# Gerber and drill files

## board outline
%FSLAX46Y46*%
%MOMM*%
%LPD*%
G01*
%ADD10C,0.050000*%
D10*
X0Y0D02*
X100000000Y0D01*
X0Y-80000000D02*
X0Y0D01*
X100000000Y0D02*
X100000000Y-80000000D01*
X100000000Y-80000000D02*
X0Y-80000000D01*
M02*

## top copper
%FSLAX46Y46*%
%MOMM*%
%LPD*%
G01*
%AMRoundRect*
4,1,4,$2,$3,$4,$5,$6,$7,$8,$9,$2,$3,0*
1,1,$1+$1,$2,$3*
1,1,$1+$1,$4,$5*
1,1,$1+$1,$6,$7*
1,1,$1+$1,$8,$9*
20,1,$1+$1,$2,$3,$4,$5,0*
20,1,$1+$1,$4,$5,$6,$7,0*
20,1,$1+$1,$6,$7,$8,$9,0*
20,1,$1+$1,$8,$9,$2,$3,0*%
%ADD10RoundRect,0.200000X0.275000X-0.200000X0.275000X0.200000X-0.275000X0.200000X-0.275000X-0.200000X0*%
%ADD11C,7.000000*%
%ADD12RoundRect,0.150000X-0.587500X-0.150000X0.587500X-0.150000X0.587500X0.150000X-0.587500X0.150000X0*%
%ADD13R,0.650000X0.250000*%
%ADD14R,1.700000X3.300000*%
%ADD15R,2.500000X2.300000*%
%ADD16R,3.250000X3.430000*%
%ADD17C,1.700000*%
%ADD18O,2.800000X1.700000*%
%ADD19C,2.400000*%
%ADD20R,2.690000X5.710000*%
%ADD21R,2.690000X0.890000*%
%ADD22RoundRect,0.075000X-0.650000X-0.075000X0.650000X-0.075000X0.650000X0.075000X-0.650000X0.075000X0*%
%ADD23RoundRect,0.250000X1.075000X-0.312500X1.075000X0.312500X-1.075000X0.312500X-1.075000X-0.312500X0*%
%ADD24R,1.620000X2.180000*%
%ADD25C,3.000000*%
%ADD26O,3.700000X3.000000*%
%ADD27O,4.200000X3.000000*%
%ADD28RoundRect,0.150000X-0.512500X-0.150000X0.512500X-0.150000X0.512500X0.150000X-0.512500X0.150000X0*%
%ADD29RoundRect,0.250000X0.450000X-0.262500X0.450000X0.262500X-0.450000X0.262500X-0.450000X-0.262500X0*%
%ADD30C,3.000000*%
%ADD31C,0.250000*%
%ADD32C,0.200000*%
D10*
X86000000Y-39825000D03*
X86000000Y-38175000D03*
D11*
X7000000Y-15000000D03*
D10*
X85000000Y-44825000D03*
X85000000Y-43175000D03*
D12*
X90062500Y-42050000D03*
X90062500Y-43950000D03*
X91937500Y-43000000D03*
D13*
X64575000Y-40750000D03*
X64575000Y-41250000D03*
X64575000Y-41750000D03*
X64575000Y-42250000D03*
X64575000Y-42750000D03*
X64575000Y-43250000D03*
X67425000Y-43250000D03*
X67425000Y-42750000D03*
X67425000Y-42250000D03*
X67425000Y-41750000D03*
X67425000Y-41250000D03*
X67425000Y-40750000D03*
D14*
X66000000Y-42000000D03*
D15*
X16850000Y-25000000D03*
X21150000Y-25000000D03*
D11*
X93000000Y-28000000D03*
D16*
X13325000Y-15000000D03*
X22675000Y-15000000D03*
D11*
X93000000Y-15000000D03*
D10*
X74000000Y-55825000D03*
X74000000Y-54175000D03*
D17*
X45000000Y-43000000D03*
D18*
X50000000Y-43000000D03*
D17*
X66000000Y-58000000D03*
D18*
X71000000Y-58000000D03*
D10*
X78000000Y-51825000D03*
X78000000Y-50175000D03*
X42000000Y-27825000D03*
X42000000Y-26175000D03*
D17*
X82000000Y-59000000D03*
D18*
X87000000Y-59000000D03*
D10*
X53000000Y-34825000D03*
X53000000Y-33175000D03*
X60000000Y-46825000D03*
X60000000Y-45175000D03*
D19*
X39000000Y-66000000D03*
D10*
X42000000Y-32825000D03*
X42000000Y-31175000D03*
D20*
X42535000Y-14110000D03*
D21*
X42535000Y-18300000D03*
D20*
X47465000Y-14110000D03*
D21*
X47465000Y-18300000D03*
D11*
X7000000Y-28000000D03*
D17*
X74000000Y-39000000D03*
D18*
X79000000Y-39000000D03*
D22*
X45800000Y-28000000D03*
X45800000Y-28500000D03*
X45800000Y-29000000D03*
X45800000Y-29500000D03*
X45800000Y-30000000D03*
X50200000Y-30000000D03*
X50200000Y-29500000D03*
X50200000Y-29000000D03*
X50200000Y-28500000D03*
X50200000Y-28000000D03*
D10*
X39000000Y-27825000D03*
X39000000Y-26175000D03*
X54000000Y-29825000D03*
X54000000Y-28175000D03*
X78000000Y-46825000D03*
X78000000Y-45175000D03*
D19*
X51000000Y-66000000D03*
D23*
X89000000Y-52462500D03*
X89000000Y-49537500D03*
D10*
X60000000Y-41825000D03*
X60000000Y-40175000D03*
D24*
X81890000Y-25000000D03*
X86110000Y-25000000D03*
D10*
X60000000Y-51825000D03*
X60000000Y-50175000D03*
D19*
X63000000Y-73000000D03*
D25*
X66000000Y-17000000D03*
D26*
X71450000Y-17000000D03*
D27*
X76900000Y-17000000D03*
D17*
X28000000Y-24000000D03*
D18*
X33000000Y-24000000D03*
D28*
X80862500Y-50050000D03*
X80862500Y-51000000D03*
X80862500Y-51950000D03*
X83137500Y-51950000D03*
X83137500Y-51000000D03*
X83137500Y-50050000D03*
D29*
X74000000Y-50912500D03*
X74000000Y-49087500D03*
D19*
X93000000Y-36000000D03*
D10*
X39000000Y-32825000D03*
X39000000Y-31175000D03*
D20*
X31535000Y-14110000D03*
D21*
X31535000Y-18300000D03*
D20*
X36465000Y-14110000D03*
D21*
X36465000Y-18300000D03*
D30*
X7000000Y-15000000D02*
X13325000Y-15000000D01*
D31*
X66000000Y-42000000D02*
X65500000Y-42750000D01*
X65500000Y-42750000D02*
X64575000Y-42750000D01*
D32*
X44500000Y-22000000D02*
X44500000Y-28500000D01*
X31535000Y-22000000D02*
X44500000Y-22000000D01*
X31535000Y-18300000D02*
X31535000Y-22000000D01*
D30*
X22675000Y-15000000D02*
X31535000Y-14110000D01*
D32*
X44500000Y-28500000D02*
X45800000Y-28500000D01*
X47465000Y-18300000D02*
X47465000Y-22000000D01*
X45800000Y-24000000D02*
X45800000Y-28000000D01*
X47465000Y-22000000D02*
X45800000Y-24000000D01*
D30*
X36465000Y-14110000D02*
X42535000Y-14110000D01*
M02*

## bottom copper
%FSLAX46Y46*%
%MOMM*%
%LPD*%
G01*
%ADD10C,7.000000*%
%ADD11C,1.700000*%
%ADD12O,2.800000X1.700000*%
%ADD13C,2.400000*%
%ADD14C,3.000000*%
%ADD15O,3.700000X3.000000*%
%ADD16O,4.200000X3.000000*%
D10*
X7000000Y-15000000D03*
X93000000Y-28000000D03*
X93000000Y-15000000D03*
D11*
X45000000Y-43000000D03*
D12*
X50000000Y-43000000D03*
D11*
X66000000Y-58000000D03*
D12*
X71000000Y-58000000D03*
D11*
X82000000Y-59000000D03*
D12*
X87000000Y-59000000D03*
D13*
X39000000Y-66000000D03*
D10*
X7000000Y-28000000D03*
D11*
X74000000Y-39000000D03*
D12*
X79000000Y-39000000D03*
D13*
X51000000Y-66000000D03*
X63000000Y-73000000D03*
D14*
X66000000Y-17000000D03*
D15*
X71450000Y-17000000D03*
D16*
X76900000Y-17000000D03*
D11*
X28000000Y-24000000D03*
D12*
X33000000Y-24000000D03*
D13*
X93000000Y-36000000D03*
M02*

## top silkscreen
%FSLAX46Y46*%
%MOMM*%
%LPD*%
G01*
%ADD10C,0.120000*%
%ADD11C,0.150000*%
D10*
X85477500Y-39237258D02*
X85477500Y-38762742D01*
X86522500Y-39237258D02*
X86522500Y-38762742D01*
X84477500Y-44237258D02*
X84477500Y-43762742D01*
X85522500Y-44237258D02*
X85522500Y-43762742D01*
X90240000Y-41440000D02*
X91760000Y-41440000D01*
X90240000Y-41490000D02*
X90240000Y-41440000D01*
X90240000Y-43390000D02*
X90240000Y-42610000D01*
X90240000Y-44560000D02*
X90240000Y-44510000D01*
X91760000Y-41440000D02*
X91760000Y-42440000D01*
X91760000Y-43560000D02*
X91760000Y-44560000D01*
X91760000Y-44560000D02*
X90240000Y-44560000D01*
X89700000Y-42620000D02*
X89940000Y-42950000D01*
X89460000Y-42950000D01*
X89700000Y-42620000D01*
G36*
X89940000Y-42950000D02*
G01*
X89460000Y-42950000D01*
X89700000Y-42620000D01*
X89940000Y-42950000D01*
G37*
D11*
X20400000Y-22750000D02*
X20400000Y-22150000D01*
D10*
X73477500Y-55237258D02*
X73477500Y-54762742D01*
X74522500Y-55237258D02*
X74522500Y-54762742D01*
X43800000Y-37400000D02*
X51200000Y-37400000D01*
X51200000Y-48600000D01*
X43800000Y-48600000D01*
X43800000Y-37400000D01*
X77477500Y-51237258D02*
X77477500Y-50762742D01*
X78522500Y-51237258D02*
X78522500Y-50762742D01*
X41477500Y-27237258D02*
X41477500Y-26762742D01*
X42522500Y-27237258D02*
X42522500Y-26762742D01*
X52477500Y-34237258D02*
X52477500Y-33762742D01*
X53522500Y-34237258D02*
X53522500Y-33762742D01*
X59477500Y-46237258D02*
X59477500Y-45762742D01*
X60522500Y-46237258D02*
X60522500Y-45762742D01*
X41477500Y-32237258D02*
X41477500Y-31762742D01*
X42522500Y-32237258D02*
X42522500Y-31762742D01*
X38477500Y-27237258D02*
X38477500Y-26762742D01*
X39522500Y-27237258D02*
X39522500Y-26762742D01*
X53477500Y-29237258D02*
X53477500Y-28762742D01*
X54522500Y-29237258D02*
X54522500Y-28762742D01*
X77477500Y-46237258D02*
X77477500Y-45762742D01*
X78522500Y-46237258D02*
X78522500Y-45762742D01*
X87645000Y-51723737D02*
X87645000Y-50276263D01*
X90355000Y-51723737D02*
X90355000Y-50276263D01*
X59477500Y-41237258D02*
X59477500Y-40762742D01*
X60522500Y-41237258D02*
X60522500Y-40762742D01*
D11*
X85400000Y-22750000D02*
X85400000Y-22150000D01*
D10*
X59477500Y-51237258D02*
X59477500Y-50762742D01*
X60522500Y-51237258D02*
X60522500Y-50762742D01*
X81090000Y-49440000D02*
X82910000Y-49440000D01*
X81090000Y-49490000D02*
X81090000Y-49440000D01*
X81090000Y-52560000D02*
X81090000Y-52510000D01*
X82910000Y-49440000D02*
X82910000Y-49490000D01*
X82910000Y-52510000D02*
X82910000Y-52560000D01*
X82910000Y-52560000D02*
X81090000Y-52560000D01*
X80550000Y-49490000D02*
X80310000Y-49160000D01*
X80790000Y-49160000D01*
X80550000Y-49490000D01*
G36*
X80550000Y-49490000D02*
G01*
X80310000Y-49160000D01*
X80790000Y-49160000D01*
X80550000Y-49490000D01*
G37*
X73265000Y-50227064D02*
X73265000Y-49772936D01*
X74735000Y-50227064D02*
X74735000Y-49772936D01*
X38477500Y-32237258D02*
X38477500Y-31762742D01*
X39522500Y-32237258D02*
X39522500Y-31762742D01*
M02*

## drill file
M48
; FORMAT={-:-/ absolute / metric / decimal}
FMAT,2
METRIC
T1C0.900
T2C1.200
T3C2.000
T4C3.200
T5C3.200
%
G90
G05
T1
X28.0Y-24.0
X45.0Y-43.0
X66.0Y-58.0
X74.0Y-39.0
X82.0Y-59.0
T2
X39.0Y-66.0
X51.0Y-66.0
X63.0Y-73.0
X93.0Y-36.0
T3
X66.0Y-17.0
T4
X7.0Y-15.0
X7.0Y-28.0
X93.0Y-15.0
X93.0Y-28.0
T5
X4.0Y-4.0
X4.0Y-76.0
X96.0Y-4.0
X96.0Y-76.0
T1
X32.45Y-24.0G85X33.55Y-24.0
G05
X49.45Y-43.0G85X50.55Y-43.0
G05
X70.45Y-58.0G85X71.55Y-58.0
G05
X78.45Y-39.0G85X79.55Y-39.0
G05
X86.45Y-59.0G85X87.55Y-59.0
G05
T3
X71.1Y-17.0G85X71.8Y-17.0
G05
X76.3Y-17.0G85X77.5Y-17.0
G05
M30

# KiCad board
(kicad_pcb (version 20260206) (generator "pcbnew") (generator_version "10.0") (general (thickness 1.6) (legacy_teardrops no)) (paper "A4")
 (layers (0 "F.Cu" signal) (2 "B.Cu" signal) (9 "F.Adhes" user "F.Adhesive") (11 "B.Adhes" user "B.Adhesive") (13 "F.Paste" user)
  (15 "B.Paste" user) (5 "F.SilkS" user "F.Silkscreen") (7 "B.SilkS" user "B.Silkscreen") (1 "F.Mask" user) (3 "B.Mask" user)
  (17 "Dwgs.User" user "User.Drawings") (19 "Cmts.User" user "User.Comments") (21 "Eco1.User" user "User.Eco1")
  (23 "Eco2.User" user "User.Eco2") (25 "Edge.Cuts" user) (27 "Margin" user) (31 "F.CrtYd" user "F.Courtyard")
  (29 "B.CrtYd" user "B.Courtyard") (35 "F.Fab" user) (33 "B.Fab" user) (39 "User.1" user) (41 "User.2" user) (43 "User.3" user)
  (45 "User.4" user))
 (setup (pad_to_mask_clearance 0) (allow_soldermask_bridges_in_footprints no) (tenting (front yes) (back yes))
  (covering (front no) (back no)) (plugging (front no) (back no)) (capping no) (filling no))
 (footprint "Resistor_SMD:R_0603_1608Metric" (layer "F.Cu") (at 86 39 90)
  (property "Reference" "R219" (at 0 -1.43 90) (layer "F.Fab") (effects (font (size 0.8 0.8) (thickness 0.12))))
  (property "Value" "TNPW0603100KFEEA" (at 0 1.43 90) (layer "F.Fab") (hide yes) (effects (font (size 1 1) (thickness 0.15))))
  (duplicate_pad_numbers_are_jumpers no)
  (fp_line (start -0.237258 -0.5225) (end 0.237258 -0.5225) (stroke (width 0.12) (type solid)) (layer "F.SilkS"))
  (fp_line (start -0.237258 0.5225) (end 0.237258 0.5225) (stroke (width 0.12) (type solid)) (layer "F.SilkS"))
  (pad "1" smd roundrect (at -0.825 0 90) (size 0.8 0.95) (layers "F.Cu" "F.Mask" "F.Paste") (roundrect_rratio 0.25)
   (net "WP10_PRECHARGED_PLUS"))
  (pad "2" smd roundrect (at 0.825 0 90) (size 0.8 0.95) (layers "F.Cu" "F.Mask" "F.Paste") (roundrect_rratio 0.25) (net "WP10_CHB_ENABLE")))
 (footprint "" (layer "F.Cu") (at 7 15)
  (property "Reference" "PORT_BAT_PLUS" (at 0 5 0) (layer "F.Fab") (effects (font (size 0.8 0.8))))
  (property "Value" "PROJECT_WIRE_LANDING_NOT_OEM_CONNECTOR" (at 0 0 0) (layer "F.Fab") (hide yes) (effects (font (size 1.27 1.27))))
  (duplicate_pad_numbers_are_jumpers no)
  (pad "1" thru_hole circle (at 0 0) (size 7 7) (drill 3.2) (layers "*.Cu" "*.Mask") (remove_unused_layers no)
   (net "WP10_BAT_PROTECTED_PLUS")))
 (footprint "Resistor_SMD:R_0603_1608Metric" (layer "F.Cu") (at 85 44 90)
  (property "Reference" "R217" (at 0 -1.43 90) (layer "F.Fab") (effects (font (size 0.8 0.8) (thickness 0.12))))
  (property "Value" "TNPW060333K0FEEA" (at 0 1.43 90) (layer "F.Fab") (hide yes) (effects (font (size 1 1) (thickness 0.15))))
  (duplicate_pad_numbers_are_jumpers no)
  (fp_line (start -0.237258 -0.5225) (end 0.237258 -0.5225) (stroke (width 0.12) (type solid)) (layer "F.SilkS"))
  (fp_line (start -0.237258 0.5225) (end 0.237258 0.5225) (stroke (width 0.12) (type solid)) (layer "F.SilkS"))
  (pad "1" smd roundrect (at -0.825 0 90) (size 0.8 0.95) (layers "F.Cu" "F.Mask" "F.Paste") (roundrect_rratio 0.25)
   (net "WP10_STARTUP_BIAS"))
  (pad "2" smd roundrect (at 0.825 0 90) (size 0.8 0.95) (layers "F.Cu" "F.Mask" "F.Paste") (roundrect_rratio 0.25)
   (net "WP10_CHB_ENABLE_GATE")))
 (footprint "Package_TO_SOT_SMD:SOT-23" (layer "F.Cu") (at 91 43)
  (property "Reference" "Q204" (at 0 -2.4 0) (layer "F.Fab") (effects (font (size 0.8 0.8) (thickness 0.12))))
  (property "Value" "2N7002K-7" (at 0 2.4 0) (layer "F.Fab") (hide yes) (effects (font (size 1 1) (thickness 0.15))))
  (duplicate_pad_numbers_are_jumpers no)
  (fp_line (start -0.76 -1.56) (end 0.76 -1.56) (stroke (width 0.12) (type solid)) (layer "F.SilkS"))
  (fp_line (start -0.76 -1.51) (end -0.76 -1.56) (stroke (width 0.12) (type solid)) (layer "F.SilkS"))
  (fp_line (start -0.76 0.39) (end -0.76 -0.39) (stroke (width 0.12) (type solid)) (layer "F.SilkS"))
  (fp_line (start -0.76 1.56) (end -0.76 1.51) (stroke (width 0.12) (type solid)) (layer "F.SilkS"))
  (fp_line (start 0.76 -1.56) (end 0.76 -0.56) (stroke (width 0.12) (type solid)) (layer "F.SilkS"))
  (fp_line (start 0.76 0.56) (end 0.76 1.56) (stroke (width 0.12) (type solid)) (layer "F.SilkS"))
  (fp_line (start 0.76 1.56) (end -0.76 1.56) (stroke (width 0.12) (type solid)) (layer "F.SilkS"))
  (fp_poly (pts (xy -1.3 -0.38) (xy -1.06 -0.05) (xy -1.54 -0.05)) (stroke (width 0.12) (type solid)) (fill yes) (layer "F.SilkS"))
  (pad "1" smd roundrect (at -0.9375 -0.95) (size 1.475 0.6) (layers "F.Cu" "F.Mask" "F.Paste") (roundrect_rratio 0.25)
   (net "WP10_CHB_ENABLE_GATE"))
  (pad "2" smd roundrect (at -0.9375 0.95) (size 1.475 0.6) (layers "F.Cu" "F.Mask" "F.Paste") (roundrect_rratio 0.25)
   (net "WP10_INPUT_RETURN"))
  (pad "3" smd roundrect (at 0.9375 0) (size 1.475 0.6) (layers "F.Cu" "F.Mask" "F.Paste") (roundrect_rratio 0.25) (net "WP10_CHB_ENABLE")))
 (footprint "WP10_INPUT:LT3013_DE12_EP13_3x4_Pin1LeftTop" (layer "F.Cu") (at 66 42)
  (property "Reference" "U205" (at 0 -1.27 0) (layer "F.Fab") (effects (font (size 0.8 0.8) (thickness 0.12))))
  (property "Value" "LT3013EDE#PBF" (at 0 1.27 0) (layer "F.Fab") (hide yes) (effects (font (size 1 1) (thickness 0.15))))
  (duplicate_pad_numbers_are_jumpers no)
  (pad "1" smd rect (at -1.425 -1.25) (size 0.65 0.25) (layers "F.Cu" "F.Mask" "F.Paste"))
  (pad "2" smd rect (at -1.425 -0.75) (size 0.65 0.25) (layers "F.Cu" "F.Mask" "F.Paste") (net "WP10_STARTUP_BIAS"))
  (pad "3" smd rect (at -1.425 -0.25) (size 0.65 0.25) (layers "F.Cu" "F.Mask" "F.Paste") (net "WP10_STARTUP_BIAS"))
  (pad "4" smd rect (at -1.425 0.25) (size 0.65 0.25) (layers "F.Cu" "F.Mask" "F.Paste") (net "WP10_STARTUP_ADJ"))
  (pad "5" smd rect (at -1.425 0.75) (size 0.65 0.25) (layers "F.Cu" "F.Mask" "F.Paste") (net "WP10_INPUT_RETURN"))
  (pad "6" smd rect (at -1.425 1.25) (size 0.65 0.25) (layers "F.Cu" "F.Mask" "F.Paste"))
  (pad "7" smd rect (at 1.425 1.25) (size 0.65 0.25) (layers "F.Cu" "F.Mask" "F.Paste") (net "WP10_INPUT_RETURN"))
  (pad "8" smd rect (at 1.425 0.75) (size 0.65 0.25) (layers "F.Cu" "F.Mask" "F.Paste") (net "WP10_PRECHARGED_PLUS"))
  (pad "9" smd rect (at 1.425 0.25) (size 0.65 0.25) (layers "F.Cu" "F.Mask" "F.Paste"))
  (pad "10" smd rect (at 1.425 -0.25) (size 0.65 0.25) (layers "F.Cu" "F.Mask" "F.Paste") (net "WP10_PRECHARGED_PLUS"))
  (pad "11" smd rect (at 1.425 -0.75) (size 0.65 0.25) (layers "F.Cu" "F.Mask" "F.Paste") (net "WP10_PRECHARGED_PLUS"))
  (pad "12" smd rect (at 1.425 -1.25) (size 0.65 0.25) (layers "F.Cu" "F.Mask" "F.Paste"))
  (pad "13" smd rect (at 0 0) (size 1.7 3.3) (layers "F.Cu" "F.Mask" "F.Paste") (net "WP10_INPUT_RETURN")))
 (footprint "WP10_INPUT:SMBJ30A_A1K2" (layer "F.Cu") (at 19 25)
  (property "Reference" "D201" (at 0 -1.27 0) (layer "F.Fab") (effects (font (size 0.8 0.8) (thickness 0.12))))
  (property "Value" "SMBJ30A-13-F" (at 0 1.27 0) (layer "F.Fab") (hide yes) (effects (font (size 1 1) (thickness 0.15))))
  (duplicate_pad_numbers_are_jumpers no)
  (fp_line (start 1.4 -2.25) (end 1.4 -2.85) (stroke (width 0.15) (type default)) (layer "F.SilkS"))
  (pad "1" smd rect (at -2.15 0) (size 2.5 2.3) (layers "F.Cu" "F.Mask" "F.Paste") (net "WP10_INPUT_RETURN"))
  (pad "2" smd rect (at 2.15 0) (size 2.5 2.3) (layers "F.Cu" "F.Mask" "F.Paste") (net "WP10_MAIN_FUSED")))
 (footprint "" (layer "F.Cu") (at 93 28)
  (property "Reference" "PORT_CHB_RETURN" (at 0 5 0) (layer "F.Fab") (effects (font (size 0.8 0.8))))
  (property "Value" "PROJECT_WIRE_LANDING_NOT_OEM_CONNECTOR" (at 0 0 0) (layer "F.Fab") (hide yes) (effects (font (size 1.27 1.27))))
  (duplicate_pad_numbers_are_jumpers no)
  (pad "1" thru_hole circle (at 0 0) (size 7 7) (drill 3.2) (layers "*.Cu" "*.Mask") (remove_unused_layers no) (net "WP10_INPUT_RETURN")))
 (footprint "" (layer "F.Cu") (at 4 4)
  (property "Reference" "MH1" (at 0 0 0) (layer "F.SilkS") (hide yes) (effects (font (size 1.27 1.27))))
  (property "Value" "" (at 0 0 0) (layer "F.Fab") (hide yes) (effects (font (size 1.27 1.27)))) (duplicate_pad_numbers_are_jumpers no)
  (pad "" np_thru_hole circle (at 0 0) (size 3.2 3.2) (drill 3.2) (layers "*.Cu" "*.Mask")))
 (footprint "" (layer "F.Cu") (at 4 76)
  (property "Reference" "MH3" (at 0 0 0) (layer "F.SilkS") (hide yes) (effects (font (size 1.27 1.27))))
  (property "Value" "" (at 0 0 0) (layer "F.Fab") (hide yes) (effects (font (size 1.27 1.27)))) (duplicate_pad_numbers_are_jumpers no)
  (pad "" np_thru_hole circle (at 0 0) (size 3.2 3.2) (drill 3.2) (layers "*.Cu" "*.Mask")))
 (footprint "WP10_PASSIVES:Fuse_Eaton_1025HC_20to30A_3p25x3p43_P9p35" (layer "F.Cu") (at 18 15)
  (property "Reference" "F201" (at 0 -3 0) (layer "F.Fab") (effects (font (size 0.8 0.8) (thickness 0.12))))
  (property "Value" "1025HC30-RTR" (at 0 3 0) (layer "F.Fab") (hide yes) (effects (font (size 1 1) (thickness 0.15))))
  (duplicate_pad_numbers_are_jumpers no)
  (pad "1" smd rect (at -4.675 0) (size 3.25 3.43) (layers "F.Cu" "F.Mask" "F.Paste") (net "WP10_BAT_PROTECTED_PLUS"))
  (pad "2" smd rect (at 4.675 0) (size 3.25 3.43) (layers "F.Cu" "F.Mask" "F.Paste") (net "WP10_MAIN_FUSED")))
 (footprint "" (layer "F.Cu") (at 93 15)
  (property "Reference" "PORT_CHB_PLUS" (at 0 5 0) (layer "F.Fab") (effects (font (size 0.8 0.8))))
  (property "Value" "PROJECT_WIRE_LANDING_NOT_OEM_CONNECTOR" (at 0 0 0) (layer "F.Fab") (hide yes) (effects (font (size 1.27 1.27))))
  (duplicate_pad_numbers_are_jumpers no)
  (pad "1" thru_hole circle (at 0 0) (size 7 7) (drill 3.2) (layers "*.Cu" "*.Mask") (remove_unused_layers no) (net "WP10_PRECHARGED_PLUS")))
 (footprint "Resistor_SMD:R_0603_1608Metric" (layer "F.Cu") (at 74 55 90)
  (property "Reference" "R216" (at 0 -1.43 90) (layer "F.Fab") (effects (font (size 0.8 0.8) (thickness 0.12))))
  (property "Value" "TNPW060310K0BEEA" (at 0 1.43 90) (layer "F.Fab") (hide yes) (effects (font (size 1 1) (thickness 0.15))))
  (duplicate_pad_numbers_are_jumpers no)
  (fp_line (start -0.237258 -0.5225) (end 0.237258 -0.5225) (stroke (width 0.12) (type solid)) (layer "F.SilkS"))
  (fp_line (start -0.237258 0.5225) (end 0.237258 0.5225) (stroke (width 0.12) (type solid)) (layer "F.SilkS"))
  (pad "1" smd roundrect (at -0.825 0 90) (size 0.8 0.95) (layers "F.Cu" "F.Mask" "F.Paste") (roundrect_rratio 0.25)
   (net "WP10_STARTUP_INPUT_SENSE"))
  (pad "2" smd roundrect (at 0.825 0 90) (size 0.8 0.95) (layers "F.Cu" "F.Mask" "F.Paste") (roundrect_rratio 0.25)
   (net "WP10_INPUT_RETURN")))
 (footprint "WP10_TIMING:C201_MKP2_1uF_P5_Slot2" (layer "F.Cu") (at 45 43)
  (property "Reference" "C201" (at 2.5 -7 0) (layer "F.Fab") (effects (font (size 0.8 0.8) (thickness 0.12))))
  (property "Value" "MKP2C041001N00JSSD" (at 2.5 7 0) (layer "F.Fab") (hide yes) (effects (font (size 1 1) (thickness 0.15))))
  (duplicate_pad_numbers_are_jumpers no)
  (fp_rect (start -1.2 -5.6) (end 6.2 5.6) (stroke (width 0.12) (type default)) (fill no) (layer "F.SilkS"))
  (pad "1" thru_hole circle (at 0 0) (size 1.7 1.7) (drill 0.9) (layers "*.Cu" "*.Mask") (remove_unused_layers no) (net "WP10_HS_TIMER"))
  (pad "2" thru_hole oval (at 5 0) (size 2.8 1.7) (drill oval 2 0.9) (layers "*.Cu" "*.Mask") (remove_unused_layers no)
   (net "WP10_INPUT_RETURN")))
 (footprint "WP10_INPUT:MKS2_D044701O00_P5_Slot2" (layer "F.Cu") (at 66 58)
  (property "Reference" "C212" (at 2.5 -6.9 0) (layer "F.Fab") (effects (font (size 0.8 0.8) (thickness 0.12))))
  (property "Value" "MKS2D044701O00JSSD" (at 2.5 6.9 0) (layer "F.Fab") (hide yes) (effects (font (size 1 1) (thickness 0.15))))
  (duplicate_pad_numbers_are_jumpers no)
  (pad "1" thru_hole circle (at 0 0) (size 1.7 1.7) (drill 0.9) (layers "*.Cu" "*.Mask") (remove_unused_layers no) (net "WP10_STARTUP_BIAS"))
  (pad "2" thru_hole oval (at 5 0) (size 2.8 1.7) (drill oval 2 0.9) (layers "*.Cu" "*.Mask") (remove_unused_layers no)
   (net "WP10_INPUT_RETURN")))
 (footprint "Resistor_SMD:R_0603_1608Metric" (layer "F.Cu") (at 78 51 90)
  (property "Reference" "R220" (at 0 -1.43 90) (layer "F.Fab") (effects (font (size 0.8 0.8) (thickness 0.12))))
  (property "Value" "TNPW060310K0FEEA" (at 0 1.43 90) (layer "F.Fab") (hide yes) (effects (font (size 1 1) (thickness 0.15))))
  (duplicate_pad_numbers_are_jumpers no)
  (fp_line (start -0.237258 -0.5225) (end 0.237258 -0.5225) (stroke (width 0.12) (type solid)) (layer "F.SilkS"))
  (fp_line (start -0.237258 0.5225) (end 0.237258 0.5225) (stroke (width 0.12) (type solid)) (layer "F.SilkS"))
  (pad "1" smd roundrect (at -0.825 0 90) (size 0.8 0.95) (layers "F.Cu" "F.Mask" "F.Paste") (roundrect_rratio 0.25)
   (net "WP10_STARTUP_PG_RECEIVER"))
  (pad "2" smd roundrect (at 0.825 0 90) (size 0.8 0.95) (layers "F.Cu" "F.Mask" "F.Paste") (roundrect_rratio 0.25)
   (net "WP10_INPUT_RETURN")))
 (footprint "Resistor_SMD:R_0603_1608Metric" (layer "F.Cu") (at 42 27 90)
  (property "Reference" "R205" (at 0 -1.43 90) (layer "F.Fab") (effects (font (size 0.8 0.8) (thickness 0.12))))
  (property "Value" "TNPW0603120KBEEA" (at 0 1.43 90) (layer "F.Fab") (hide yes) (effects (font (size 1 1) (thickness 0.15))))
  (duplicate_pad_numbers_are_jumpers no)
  (fp_line (start -0.237258 -0.5225) (end 0.237258 -0.5225) (stroke (width 0.12) (type solid)) (layer "F.SilkS"))
  (fp_line (start -0.237258 0.5225) (end 0.237258 0.5225) (stroke (width 0.12) (type solid)) (layer "F.SilkS"))
  (pad "1" smd roundrect (at -0.825 0 90) (size 0.8 0.95) (layers "F.Cu" "F.Mask" "F.Paste") (roundrect_rratio 0.25) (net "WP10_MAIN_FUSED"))
  (pad "2" smd roundrect (at 0.825 0 90) (size 0.8 0.95) (layers "F.Cu" "F.Mask" "F.Paste") (roundrect_rratio 0.25) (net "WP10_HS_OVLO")))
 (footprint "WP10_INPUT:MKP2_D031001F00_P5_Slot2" (layer "F.Cu") (at 82 59)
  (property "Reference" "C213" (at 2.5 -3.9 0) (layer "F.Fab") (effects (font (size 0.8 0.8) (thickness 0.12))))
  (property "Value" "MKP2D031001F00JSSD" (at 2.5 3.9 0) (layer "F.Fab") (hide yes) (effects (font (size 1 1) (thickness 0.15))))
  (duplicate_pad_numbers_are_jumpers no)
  (pad "1" thru_hole circle (at 0 0) (size 1.7 1.7) (drill 0.9) (layers "*.Cu" "*.Mask") (remove_unused_layers no) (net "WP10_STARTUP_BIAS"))
  (pad "2" thru_hole oval (at 5 0) (size 2.8 1.7) (drill oval 2 0.9) (layers "*.Cu" "*.Mask") (remove_unused_layers no)
   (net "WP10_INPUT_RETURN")))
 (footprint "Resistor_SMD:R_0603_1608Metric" (layer "F.Cu") (at 53 34 90)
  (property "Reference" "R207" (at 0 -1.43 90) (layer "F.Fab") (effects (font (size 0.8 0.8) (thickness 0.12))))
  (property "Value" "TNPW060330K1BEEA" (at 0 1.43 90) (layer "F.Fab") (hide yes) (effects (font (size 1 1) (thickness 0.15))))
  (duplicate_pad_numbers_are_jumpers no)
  (fp_line (start -0.237258 -0.5225) (end 0.237258 -0.5225) (stroke (width 0.12) (type solid)) (layer "F.SilkS"))
  (fp_line (start -0.237258 0.5225) (end 0.237258 0.5225) (stroke (width 0.12) (type solid)) (layer "F.SilkS"))
  (pad "1" smd roundrect (at -0.825 0 90) (size 0.8 0.95) (layers "F.Cu" "F.Mask" "F.Paste") (roundrect_rratio 0.25)
   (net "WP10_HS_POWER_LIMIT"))
  (pad "2" smd roundrect (at 0.825 0 90) (size 0.8 0.95) (layers "F.Cu" "F.Mask" "F.Paste") (roundrect_rratio 0.25)
   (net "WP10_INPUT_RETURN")))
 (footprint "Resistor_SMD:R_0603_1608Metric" (layer "F.Cu") (at 60 46 90)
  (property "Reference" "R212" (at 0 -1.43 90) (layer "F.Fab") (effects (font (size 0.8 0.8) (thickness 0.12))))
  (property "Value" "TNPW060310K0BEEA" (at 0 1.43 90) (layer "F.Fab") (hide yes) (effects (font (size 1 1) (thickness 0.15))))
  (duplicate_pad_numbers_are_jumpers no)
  (fp_line (start -0.237258 -0.5225) (end 0.237258 -0.5225) (stroke (width 0.12) (type solid)) (layer "F.SilkS"))
  (fp_line (start -0.237258 0.5225) (end 0.237258 0.5225) (stroke (width 0.12) (type solid)) (layer "F.SilkS"))
  (pad "1" smd roundrect (at -0.825 0 90) (size 0.8 0.95) (layers "F.Cu" "F.Mask" "F.Paste") (roundrect_rratio 0.25)
   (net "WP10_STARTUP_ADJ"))
  (pad "2" smd roundrect (at 0.825 0 90) (size 0.8 0.95) (layers "F.Cu" "F.Mask" "F.Paste") (roundrect_rratio 0.25)
   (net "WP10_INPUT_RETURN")))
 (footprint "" (layer "F.Cu") (at 39 66)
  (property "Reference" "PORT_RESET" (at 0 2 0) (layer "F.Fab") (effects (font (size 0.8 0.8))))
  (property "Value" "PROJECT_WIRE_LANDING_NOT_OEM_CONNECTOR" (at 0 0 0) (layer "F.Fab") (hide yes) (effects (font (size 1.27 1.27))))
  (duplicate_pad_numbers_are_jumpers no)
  (pad "1" thru_hole circle (at 0 0) (size 2.4 2.4) (drill 1.2) (layers "*.Cu" "*.Mask") (remove_unused_layers no) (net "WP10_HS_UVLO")))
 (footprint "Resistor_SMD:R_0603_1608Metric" (layer "F.Cu") (at 42 32 90)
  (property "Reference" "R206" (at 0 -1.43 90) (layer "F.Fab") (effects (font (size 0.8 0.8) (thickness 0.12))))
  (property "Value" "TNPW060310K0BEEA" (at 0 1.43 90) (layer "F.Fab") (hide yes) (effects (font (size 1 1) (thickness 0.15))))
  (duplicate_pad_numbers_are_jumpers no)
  (fp_line (start -0.237258 -0.5225) (end 0.237258 -0.5225) (stroke (width 0.12) (type solid)) (layer "F.SilkS"))
  (fp_line (start -0.237258 0.5225) (end 0.237258 0.5225) (stroke (width 0.12) (type solid)) (layer "F.SilkS"))
  (pad "1" smd roundrect (at -0.825 0 90) (size 0.8 0.95) (layers "F.Cu" "F.Mask" "F.Paste") (roundrect_rratio 0.25) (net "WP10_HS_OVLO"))
  (pad "2" smd roundrect (at 0.825 0 90) (size 0.8 0.95) (layers "F.Cu" "F.Mask" "F.Paste") (roundrect_rratio 0.25)
   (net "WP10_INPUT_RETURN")))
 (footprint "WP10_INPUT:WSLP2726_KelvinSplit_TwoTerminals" (layer "F.Cu") (at 45 15)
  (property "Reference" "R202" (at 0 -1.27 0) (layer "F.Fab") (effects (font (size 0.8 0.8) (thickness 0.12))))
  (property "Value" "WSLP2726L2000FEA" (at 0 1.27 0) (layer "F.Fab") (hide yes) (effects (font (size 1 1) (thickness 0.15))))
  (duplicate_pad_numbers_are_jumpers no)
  (pad "1" smd rect (at -2.465 -0.89) (size 2.69 5.71) (layers "F.Cu" "F.Mask" "F.Paste") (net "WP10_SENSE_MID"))
  (pad "1" smd rect (at -2.465 3.3) (size 2.69 0.89) (layers "F.Cu" "F.Mask" "F.Paste") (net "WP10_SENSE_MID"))
  (pad "2" smd rect (at 2.465 -0.89) (size 2.69 5.71) (layers "F.Cu" "F.Mask" "F.Paste") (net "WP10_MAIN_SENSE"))
  (pad "2" smd rect (at 2.465 3.3) (size 2.69 0.89) (layers "F.Cu" "F.Mask" "F.Paste") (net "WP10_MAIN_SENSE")))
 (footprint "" (layer "F.Cu") (at 7 28)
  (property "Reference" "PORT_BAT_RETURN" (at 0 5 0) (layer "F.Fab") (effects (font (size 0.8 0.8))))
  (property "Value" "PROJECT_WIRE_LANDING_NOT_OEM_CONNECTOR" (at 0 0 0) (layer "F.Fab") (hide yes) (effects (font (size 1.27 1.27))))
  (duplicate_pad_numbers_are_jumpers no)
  (pad "1" thru_hole circle (at 0 0) (size 7 7) (drill 3.2) (layers "*.Cu" "*.Mask") (remove_unused_layers no) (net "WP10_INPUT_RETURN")))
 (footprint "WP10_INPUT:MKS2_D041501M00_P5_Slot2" (layer "F.Cu") (at 74 39)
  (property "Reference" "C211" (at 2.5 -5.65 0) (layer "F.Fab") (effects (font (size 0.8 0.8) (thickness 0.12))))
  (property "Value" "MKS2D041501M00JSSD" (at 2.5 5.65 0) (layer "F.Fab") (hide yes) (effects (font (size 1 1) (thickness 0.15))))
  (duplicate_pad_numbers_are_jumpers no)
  (pad "1" thru_hole circle (at 0 0) (size 1.7 1.7) (drill 0.9) (layers "*.Cu" "*.Mask") (remove_unused_layers no)
   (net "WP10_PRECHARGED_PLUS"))
  (pad "2" thru_hole oval (at 5 0) (size 2.8 1.7) (drill oval 2 0.9) (layers "*.Cu" "*.Mask") (remove_unused_layers no)
   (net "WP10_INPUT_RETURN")))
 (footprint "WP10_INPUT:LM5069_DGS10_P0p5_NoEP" (layer "F.Cu") (at 48 29)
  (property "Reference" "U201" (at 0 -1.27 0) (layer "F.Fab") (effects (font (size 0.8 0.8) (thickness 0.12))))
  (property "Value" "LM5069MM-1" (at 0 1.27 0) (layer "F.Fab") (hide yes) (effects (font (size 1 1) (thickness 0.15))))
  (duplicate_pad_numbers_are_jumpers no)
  (pad "1" smd roundrect (at -2.2 -1) (size 1.45 0.3) (layers "F.Cu" "F.Mask" "F.Paste") (roundrect_rratio 0.25) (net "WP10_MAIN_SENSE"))
  (pad "2" smd roundrect (at -2.2 -0.5) (size 1.45 0.3) (layers "F.Cu" "F.Mask" "F.Paste") (roundrect_rratio 0.25) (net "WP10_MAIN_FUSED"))
  (pad "3" smd roundrect (at -2.2 0) (size 1.45 0.3) (layers "F.Cu" "F.Mask" "F.Paste") (roundrect_rratio 0.25) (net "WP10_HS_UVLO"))
  (pad "4" smd roundrect (at -2.2 0.5) (size 1.45 0.3) (layers "F.Cu" "F.Mask" "F.Paste") (roundrect_rratio 0.25) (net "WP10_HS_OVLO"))
  (pad "5" smd roundrect (at -2.2 1) (size 1.45 0.3) (layers "F.Cu" "F.Mask" "F.Paste") (roundrect_rratio 0.25) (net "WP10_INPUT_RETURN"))
  (pad "6" smd roundrect (at 2.2 1) (size 1.45 0.3) (layers "F.Cu" "F.Mask" "F.Paste") (roundrect_rratio 0.25) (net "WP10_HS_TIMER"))
  (pad "7" smd roundrect (at 2.2 0.5) (size 1.45 0.3) (layers "F.Cu" "F.Mask" "F.Paste") (roundrect_rratio 0.25) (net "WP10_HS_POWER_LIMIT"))
  (pad "8" smd roundrect (at 2.2 0) (size 1.45 0.3) (layers "F.Cu" "F.Mask" "F.Paste") (roundrect_rratio 0.25) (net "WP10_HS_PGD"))
  (pad "9" smd roundrect (at 2.2 -0.5) (size 1.45 0.3) (layers "F.Cu" "F.Mask" "F.Paste") (roundrect_rratio 0.25)
   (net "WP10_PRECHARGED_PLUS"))
  (pad "10" smd roundrect (at 2.2 -1) (size 1.45 0.3) (layers "F.Cu" "F.Mask" "F.Paste") (roundrect_rratio 0.25) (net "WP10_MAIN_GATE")))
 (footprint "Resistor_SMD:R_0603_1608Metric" (layer "F.Cu") (at 39 27 90)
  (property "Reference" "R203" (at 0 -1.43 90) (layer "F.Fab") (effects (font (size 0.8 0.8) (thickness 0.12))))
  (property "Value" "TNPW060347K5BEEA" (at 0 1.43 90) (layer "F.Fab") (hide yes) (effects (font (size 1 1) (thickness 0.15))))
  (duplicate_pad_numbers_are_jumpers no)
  (fp_line (start -0.237258 -0.5225) (end 0.237258 -0.5225) (stroke (width 0.12) (type solid)) (layer "F.SilkS"))
  (fp_line (start -0.237258 0.5225) (end 0.237258 0.5225) (stroke (width 0.12) (type solid)) (layer "F.SilkS"))
  (pad "1" smd roundrect (at -0.825 0 90) (size 0.8 0.95) (layers "F.Cu" "F.Mask" "F.Paste") (roundrect_rratio 0.25) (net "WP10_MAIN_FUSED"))
  (pad "2" smd roundrect (at 0.825 0 90) (size 0.8 0.95) (layers "F.Cu" "F.Mask" "F.Paste") (roundrect_rratio 0.25) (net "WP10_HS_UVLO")))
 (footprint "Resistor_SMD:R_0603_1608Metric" (layer "F.Cu") (at 54 29 90)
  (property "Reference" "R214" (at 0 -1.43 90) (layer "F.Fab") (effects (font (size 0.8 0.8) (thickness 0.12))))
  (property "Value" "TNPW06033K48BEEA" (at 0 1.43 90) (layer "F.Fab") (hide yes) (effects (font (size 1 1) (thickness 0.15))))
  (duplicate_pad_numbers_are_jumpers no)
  (fp_line (start -0.237258 -0.5225) (end 0.237258 -0.5225) (stroke (width 0.12) (type solid)) (layer "F.SilkS"))
  (fp_line (start -0.237258 0.5225) (end 0.237258 0.5225) (stroke (width 0.12) (type solid)) (layer "F.SilkS"))
  (pad "1" smd roundrect (at -0.825 0 90) (size 0.8 0.95) (layers "F.Cu" "F.Mask" "F.Paste") (roundrect_rratio 0.25)
   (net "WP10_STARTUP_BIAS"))
  (pad "2" smd roundrect (at 0.825 0 90) (size 0.8 0.95) (layers "F.Cu" "F.Mask" "F.Paste") (roundrect_rratio 0.25) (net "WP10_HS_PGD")))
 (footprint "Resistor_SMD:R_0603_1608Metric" (layer "F.Cu") (at 78 46 90)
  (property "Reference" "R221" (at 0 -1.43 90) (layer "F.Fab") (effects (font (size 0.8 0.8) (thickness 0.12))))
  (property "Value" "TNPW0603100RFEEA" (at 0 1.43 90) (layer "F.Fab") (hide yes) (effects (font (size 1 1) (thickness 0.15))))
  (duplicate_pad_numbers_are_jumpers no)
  (fp_line (start -0.237258 -0.5225) (end 0.237258 -0.5225) (stroke (width 0.12) (type solid)) (layer "F.SilkS"))
  (fp_line (start -0.237258 0.5225) (end 0.237258 0.5225) (stroke (width 0.12) (type solid)) (layer "F.SilkS"))
  (pad "1" smd roundrect (at -0.825 0 90) (size 0.8 0.95) (layers "F.Cu" "F.Mask" "F.Paste") (roundrect_rratio 0.25) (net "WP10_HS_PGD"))
  (pad "2" smd roundrect (at 0.825 0 90) (size 0.8 0.95) (layers "F.Cu" "F.Mask" "F.Paste") (roundrect_rratio 0.25)
   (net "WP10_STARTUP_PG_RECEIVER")))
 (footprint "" (layer "F.Cu") (at 96 4)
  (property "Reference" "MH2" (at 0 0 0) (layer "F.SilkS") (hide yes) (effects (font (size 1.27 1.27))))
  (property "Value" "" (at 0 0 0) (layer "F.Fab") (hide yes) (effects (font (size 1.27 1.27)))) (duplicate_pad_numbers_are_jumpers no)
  (pad "" np_thru_hole circle (at 0 0) (size 3.2 3.2) (drill 3.2) (layers "*.Cu" "*.Mask")))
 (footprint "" (layer "F.Cu") (at 51 66)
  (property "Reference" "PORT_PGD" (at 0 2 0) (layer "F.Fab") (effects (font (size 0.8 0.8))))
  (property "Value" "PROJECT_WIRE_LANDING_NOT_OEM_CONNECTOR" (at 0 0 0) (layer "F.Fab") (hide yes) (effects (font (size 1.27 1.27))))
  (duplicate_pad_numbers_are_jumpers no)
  (pad "1" thru_hole circle (at 0 0) (size 2.4 2.4) (drill 1.2) (layers "*.Cu" "*.Mask") (remove_unused_layers no) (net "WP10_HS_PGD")))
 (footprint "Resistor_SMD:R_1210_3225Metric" (layer "F.Cu") (at 89 51 90)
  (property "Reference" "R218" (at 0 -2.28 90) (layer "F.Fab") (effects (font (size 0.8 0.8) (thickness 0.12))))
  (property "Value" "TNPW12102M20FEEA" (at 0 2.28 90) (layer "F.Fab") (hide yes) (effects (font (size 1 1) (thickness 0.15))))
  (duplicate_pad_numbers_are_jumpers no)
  (fp_line (start -0.723737 -1.355) (end 0.723737 -1.355) (stroke (width 0.12) (type solid)) (layer "F.SilkS"))
  (fp_line (start -0.723737 1.355) (end 0.723737 1.355) (stroke (width 0.12) (type solid)) (layer "F.SilkS"))
  (pad "1" smd roundrect (at -1.4625 0 90) (size 1.125 2.65) (layers "F.Cu" "F.Mask" "F.Paste") (roundrect_rratio 0.222222)
   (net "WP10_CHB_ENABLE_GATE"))
  (pad "2" smd roundrect (at 1.4625 0 90) (size 1.125 2.65) (layers "F.Cu" "F.Mask" "F.Paste") (roundrect_rratio 0.222222)
   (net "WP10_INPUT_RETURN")))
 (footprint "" (layer "F.Cu") (at 96 76)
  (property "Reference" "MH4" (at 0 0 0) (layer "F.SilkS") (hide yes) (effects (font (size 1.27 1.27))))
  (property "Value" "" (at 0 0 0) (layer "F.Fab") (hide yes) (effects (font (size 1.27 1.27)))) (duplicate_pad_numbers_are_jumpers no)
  (pad "" np_thru_hole circle (at 0 0) (size 3.2 3.2) (drill 3.2) (layers "*.Cu" "*.Mask")))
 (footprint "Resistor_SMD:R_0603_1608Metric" (layer "F.Cu") (at 60 41 90)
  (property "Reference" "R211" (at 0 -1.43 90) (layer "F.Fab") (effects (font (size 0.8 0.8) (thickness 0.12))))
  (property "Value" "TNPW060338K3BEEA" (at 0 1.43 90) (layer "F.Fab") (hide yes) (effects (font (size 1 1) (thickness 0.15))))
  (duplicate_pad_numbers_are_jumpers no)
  (fp_line (start -0.237258 -0.5225) (end 0.237258 -0.5225) (stroke (width 0.12) (type solid)) (layer "F.SilkS"))
  (fp_line (start -0.237258 0.5225) (end 0.237258 0.5225) (stroke (width 0.12) (type solid)) (layer "F.SilkS"))
  (pad "1" smd roundrect (at -0.825 0 90) (size 0.8 0.95) (layers "F.Cu" "F.Mask" "F.Paste") (roundrect_rratio 0.25)
   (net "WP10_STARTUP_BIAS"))
  (pad "2" smd roundrect (at 0.825 0 90) (size 0.8 0.95) (layers "F.Cu" "F.Mask" "F.Paste") (roundrect_rratio 0.25) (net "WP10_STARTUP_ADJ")))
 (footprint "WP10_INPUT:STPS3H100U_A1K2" (layer "F.Cu") (at 84 25)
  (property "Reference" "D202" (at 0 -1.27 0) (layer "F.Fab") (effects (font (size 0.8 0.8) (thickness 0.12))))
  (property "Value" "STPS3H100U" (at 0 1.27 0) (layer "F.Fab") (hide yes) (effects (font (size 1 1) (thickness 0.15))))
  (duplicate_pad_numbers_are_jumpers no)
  (fp_line (start 1.4 -2.25) (end 1.4 -2.85) (stroke (width 0.15) (type default)) (layer "F.SilkS"))
  (pad "1" smd rect (at -2.11 0) (size 1.62 2.18) (layers "F.Cu" "F.Mask" "F.Paste") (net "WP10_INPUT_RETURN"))
  (pad "2" smd rect (at 2.11 0) (size 1.62 2.18) (layers "F.Cu" "F.Mask" "F.Paste") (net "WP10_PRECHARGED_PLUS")))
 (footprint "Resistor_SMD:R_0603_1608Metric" (layer "F.Cu") (at 60 51 90)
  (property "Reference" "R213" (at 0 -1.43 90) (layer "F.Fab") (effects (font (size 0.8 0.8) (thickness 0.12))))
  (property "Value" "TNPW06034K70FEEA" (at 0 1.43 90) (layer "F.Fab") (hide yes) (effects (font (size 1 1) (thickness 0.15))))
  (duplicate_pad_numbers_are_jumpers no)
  (fp_line (start -0.237258 -0.5225) (end 0.237258 -0.5225) (stroke (width 0.12) (type solid)) (layer "F.SilkS"))
  (fp_line (start -0.237258 0.5225) (end 0.237258 0.5225) (stroke (width 0.12) (type solid)) (layer "F.SilkS"))
  (pad "1" smd roundrect (at -0.825 0 90) (size 0.8 0.95) (layers "F.Cu" "F.Mask" "F.Paste") (roundrect_rratio 0.25)
   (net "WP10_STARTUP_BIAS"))
  (pad "2" smd roundrect (at 0.825 0 90) (size 0.8 0.95) (layers "F.Cu" "F.Mask" "F.Paste") (roundrect_rratio 0.25)
   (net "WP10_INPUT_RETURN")))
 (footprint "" (layer "F.Cu") (at 63 73)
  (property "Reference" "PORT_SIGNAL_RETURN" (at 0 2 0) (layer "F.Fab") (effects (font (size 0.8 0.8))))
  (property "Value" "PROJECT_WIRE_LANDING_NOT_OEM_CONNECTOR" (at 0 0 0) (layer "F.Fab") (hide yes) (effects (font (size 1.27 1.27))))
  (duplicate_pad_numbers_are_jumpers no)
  (pad "1" thru_hole circle (at 0 0) (size 2.4 2.4) (drill 1.2) (layers "*.Cu" "*.Mask") (remove_unused_layers no) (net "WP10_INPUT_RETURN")))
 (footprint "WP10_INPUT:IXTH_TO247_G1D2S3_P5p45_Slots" (layer "F.Cu") (at 66 17)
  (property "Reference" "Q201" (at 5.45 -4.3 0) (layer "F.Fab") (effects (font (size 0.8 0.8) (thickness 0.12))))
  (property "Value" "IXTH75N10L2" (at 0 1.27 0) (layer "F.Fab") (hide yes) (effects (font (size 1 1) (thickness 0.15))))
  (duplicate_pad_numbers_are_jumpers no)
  (pad "1" thru_hole circle (at 0 0) (size 3 3) (drill 2) (layers "*.Cu" "*.Mask") (remove_unused_layers no) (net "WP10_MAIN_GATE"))
  (pad "2" thru_hole oval (at 5.45 0) (size 3.7 3) (drill oval 2.7 2) (layers "*.Cu" "*.Mask") (remove_unused_layers no)
   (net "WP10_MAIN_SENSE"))
  (pad "3" thru_hole oval (at 10.9 0) (size 4.2 3) (drill oval 3.2 2) (layers "*.Cu" "*.Mask") (remove_unused_layers no)
   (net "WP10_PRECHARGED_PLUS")))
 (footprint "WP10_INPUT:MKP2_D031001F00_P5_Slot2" (layer "F.Cu") (at 28 24)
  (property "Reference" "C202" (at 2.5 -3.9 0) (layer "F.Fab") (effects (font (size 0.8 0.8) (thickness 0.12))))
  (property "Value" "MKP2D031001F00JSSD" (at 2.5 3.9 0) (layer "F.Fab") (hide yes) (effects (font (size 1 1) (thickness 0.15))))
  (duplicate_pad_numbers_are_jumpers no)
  (pad "1" thru_hole circle (at 0 0) (size 1.7 1.7) (drill 0.9) (layers "*.Cu" "*.Mask") (remove_unused_layers no) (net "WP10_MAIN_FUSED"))
  (pad "2" thru_hole oval (at 5 0) (size 2.8 1.7) (drill oval 2 0.9) (layers "*.Cu" "*.Mask") (remove_unused_layers no)
   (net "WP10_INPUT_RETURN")))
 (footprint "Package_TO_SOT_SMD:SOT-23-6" (layer "F.Cu") (at 82 51)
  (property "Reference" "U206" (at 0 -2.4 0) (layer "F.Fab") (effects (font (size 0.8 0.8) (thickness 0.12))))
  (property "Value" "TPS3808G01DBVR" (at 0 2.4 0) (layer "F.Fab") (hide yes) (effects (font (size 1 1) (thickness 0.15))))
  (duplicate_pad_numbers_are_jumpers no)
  (fp_line (start -0.91 -1.56) (end 0.91 -1.56) (stroke (width 0.12) (type solid)) (layer "F.SilkS"))
  (fp_line (start -0.91 -1.51) (end -0.91 -1.56) (stroke (width 0.12) (type solid)) (layer "F.SilkS"))
  (fp_line (start -0.91 1.56) (end -0.91 1.51) (stroke (width 0.12) (type solid)) (layer "F.SilkS"))
  (fp_line (start 0.91 -1.56) (end 0.91 -1.51) (stroke (width 0.12) (type solid)) (layer "F.SilkS"))
  (fp_line (start 0.91 1.51) (end 0.91 1.56) (stroke (width 0.12) (type solid)) (layer "F.SilkS"))
  (fp_line (start 0.91 1.56) (end -0.91 1.56) (stroke (width 0.12) (type solid)) (layer "F.SilkS"))
  (fp_poly (pts (xy -1.45 -1.51) (xy -1.69 -1.84) (xy -1.21 -1.84)) (stroke (width 0.12) (type solid)) (fill yes) (layer "F.SilkS"))
  (pad "1" smd roundrect (at -1.1375 -0.95) (size 1.325 0.6) (layers "F.Cu" "F.Mask" "F.Paste") (roundrect_rratio 0.25)
   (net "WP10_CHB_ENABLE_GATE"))
  (pad "2" smd roundrect (at -1.1375 0) (size 1.325 0.6) (layers "F.Cu" "F.Mask" "F.Paste") (roundrect_rratio 0.25)
   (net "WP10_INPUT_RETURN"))
  (pad "3" smd roundrect (at -1.1375 0.95) (size 1.325 0.6) (layers "F.Cu" "F.Mask" "F.Paste") (roundrect_rratio 0.25)
   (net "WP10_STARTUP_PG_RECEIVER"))
  (pad "4" smd roundrect (at 1.1375 0.95) (size 1.325 0.6) (layers "F.Cu" "F.Mask" "F.Paste") (roundrect_rratio 0.25))
  (pad "5" smd roundrect (at 1.1375 0) (size 1.325 0.6) (layers "F.Cu" "F.Mask" "F.Paste") (roundrect_rratio 0.25)
   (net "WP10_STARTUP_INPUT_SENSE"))
  (pad "6" smd roundrect (at 1.1375 -0.95) (size 1.325 0.6) (layers "F.Cu" "F.Mask" "F.Paste") (roundrect_rratio 0.25)
   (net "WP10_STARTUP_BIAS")))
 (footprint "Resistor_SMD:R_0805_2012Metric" (layer "F.Cu") (at 74 50 90)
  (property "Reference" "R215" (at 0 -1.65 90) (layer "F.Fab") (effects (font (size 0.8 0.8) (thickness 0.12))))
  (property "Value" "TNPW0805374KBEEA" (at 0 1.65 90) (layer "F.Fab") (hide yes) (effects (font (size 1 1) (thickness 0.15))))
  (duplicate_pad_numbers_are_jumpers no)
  (fp_line (start -0.227064 -0.735) (end 0.227064 -0.735) (stroke (width 0.12) (type solid)) (layer "F.SilkS"))
  (fp_line (start -0.227064 0.735) (end 0.227064 0.735) (stroke (width 0.12) (type solid)) (layer "F.SilkS"))
  (pad "1" smd roundrect (at -0.9125 0 90) (size 1.025 1.4) (layers "F.Cu" "F.Mask" "F.Paste") (roundrect_rratio 0.243902)
   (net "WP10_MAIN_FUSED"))
  (pad "2" smd roundrect (at 0.9125 0 90) (size 1.025 1.4) (layers "F.Cu" "F.Mask" "F.Paste") (roundrect_rratio 0.243902)
   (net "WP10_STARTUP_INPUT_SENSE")))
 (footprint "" (layer "F.Cu") (at 93 36)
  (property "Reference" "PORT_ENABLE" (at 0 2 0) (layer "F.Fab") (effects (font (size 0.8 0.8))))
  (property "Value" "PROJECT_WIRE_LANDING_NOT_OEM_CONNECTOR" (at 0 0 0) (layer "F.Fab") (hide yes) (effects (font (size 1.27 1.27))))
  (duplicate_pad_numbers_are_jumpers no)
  (pad "1" thru_hole circle (at 0 0) (size 2.4 2.4) (drill 1.2) (layers "*.Cu" "*.Mask") (remove_unused_layers no) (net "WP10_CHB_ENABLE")))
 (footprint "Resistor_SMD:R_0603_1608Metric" (layer "F.Cu") (at 39 32 90)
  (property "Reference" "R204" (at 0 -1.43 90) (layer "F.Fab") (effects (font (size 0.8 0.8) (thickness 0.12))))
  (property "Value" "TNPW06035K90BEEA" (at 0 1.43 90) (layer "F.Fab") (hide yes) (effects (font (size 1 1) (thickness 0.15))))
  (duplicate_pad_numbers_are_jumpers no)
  (fp_line (start -0.237258 -0.5225) (end 0.237258 -0.5225) (stroke (width 0.12) (type solid)) (layer "F.SilkS"))
  (fp_line (start -0.237258 0.5225) (end 0.237258 0.5225) (stroke (width 0.12) (type solid)) (layer "F.SilkS"))
  (pad "1" smd roundrect (at -0.825 0 90) (size 0.8 0.95) (layers "F.Cu" "F.Mask" "F.Paste") (roundrect_rratio 0.25) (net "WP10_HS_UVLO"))
  (pad "2" smd roundrect (at 0.825 0 90) (size 0.8 0.95) (layers "F.Cu" "F.Mask" "F.Paste") (roundrect_rratio 0.25)
   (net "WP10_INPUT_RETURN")))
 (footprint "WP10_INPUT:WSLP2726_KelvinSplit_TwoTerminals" (layer "F.Cu") (at 34 15)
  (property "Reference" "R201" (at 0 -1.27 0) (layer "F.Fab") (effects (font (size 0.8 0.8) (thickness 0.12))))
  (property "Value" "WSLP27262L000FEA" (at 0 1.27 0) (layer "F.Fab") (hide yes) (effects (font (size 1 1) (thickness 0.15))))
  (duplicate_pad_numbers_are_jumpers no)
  (pad "1" smd rect (at -2.465 -0.89) (size 2.69 5.71) (layers "F.Cu" "F.Mask" "F.Paste") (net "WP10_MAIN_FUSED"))
  (pad "1" smd rect (at -2.465 3.3) (size 2.69 0.89) (layers "F.Cu" "F.Mask" "F.Paste") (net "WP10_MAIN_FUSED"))
  (pad "2" smd rect (at 2.465 -0.89) (size 2.69 5.71) (layers "F.Cu" "F.Mask" "F.Paste") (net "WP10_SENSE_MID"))
  (pad "2" smd rect (at 2.465 3.3) (size 2.69 0.89) (layers "F.Cu" "F.Mask" "F.Paste") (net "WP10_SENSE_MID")))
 (gr_line (start 0 0) (end 100 0) (stroke (width 0.05) (type default)) (layer "Edge.Cuts"))
 (gr_line (start 0 80) (end 0 0) (stroke (width 0.05) (type default)) (layer "Edge.Cuts"))
 (gr_line (start 100 0) (end 100 80) (stroke (width 0.05) (type default)) (layer "Edge.Cuts"))
 (gr_line (start 100 80) (end 0 80) (stroke (width 0.05) (type default)) (layer "Edge.Cuts"))
 (segment (start 7 15) (end 13.325 15) (width 3) (layer "F.Cu") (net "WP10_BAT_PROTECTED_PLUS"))
 (segment (start 66 42) (end 65.5 42.75) (width 0.25) (layer "F.Cu") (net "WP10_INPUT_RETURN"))
 (segment (start 65.5 42.75) (end 64.575 42.75) (width 0.25) (layer "F.Cu") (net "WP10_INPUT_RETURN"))
 (segment (start 44.5 22) (end 44.5 28.5) (width 0.2) (layer "F.Cu") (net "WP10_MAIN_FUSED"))
 (segment (start 31.535 22) (end 44.5 22) (width 0.2) (layer "F.Cu") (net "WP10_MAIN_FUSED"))
 (segment (start 31.535 18.3) (end 31.535 22) (width 0.2) (layer "F.Cu") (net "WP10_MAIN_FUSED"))
 (segment (start 22.675 15) (end 31.535 14.11) (width 3) (layer "F.Cu") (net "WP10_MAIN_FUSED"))
 (segment (start 44.5 28.5) (end 45.8 28.5) (width 0.2) (layer "F.Cu") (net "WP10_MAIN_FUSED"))
 (segment (start 47.465 18.3) (end 47.465 22) (width 0.2) (layer "F.Cu") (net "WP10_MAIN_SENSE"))
 (segment (start 45.8 24) (end 45.8 28) (width 0.2) (layer "F.Cu") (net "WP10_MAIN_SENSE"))
 (segment (start 47.465 22) (end 45.8 24) (width 0.2) (layer "F.Cu") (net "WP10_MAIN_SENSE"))
 (segment (start 36.465 14.11) (end 42.535 14.11) (width 3) (layer "F.Cu") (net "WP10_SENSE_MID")))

